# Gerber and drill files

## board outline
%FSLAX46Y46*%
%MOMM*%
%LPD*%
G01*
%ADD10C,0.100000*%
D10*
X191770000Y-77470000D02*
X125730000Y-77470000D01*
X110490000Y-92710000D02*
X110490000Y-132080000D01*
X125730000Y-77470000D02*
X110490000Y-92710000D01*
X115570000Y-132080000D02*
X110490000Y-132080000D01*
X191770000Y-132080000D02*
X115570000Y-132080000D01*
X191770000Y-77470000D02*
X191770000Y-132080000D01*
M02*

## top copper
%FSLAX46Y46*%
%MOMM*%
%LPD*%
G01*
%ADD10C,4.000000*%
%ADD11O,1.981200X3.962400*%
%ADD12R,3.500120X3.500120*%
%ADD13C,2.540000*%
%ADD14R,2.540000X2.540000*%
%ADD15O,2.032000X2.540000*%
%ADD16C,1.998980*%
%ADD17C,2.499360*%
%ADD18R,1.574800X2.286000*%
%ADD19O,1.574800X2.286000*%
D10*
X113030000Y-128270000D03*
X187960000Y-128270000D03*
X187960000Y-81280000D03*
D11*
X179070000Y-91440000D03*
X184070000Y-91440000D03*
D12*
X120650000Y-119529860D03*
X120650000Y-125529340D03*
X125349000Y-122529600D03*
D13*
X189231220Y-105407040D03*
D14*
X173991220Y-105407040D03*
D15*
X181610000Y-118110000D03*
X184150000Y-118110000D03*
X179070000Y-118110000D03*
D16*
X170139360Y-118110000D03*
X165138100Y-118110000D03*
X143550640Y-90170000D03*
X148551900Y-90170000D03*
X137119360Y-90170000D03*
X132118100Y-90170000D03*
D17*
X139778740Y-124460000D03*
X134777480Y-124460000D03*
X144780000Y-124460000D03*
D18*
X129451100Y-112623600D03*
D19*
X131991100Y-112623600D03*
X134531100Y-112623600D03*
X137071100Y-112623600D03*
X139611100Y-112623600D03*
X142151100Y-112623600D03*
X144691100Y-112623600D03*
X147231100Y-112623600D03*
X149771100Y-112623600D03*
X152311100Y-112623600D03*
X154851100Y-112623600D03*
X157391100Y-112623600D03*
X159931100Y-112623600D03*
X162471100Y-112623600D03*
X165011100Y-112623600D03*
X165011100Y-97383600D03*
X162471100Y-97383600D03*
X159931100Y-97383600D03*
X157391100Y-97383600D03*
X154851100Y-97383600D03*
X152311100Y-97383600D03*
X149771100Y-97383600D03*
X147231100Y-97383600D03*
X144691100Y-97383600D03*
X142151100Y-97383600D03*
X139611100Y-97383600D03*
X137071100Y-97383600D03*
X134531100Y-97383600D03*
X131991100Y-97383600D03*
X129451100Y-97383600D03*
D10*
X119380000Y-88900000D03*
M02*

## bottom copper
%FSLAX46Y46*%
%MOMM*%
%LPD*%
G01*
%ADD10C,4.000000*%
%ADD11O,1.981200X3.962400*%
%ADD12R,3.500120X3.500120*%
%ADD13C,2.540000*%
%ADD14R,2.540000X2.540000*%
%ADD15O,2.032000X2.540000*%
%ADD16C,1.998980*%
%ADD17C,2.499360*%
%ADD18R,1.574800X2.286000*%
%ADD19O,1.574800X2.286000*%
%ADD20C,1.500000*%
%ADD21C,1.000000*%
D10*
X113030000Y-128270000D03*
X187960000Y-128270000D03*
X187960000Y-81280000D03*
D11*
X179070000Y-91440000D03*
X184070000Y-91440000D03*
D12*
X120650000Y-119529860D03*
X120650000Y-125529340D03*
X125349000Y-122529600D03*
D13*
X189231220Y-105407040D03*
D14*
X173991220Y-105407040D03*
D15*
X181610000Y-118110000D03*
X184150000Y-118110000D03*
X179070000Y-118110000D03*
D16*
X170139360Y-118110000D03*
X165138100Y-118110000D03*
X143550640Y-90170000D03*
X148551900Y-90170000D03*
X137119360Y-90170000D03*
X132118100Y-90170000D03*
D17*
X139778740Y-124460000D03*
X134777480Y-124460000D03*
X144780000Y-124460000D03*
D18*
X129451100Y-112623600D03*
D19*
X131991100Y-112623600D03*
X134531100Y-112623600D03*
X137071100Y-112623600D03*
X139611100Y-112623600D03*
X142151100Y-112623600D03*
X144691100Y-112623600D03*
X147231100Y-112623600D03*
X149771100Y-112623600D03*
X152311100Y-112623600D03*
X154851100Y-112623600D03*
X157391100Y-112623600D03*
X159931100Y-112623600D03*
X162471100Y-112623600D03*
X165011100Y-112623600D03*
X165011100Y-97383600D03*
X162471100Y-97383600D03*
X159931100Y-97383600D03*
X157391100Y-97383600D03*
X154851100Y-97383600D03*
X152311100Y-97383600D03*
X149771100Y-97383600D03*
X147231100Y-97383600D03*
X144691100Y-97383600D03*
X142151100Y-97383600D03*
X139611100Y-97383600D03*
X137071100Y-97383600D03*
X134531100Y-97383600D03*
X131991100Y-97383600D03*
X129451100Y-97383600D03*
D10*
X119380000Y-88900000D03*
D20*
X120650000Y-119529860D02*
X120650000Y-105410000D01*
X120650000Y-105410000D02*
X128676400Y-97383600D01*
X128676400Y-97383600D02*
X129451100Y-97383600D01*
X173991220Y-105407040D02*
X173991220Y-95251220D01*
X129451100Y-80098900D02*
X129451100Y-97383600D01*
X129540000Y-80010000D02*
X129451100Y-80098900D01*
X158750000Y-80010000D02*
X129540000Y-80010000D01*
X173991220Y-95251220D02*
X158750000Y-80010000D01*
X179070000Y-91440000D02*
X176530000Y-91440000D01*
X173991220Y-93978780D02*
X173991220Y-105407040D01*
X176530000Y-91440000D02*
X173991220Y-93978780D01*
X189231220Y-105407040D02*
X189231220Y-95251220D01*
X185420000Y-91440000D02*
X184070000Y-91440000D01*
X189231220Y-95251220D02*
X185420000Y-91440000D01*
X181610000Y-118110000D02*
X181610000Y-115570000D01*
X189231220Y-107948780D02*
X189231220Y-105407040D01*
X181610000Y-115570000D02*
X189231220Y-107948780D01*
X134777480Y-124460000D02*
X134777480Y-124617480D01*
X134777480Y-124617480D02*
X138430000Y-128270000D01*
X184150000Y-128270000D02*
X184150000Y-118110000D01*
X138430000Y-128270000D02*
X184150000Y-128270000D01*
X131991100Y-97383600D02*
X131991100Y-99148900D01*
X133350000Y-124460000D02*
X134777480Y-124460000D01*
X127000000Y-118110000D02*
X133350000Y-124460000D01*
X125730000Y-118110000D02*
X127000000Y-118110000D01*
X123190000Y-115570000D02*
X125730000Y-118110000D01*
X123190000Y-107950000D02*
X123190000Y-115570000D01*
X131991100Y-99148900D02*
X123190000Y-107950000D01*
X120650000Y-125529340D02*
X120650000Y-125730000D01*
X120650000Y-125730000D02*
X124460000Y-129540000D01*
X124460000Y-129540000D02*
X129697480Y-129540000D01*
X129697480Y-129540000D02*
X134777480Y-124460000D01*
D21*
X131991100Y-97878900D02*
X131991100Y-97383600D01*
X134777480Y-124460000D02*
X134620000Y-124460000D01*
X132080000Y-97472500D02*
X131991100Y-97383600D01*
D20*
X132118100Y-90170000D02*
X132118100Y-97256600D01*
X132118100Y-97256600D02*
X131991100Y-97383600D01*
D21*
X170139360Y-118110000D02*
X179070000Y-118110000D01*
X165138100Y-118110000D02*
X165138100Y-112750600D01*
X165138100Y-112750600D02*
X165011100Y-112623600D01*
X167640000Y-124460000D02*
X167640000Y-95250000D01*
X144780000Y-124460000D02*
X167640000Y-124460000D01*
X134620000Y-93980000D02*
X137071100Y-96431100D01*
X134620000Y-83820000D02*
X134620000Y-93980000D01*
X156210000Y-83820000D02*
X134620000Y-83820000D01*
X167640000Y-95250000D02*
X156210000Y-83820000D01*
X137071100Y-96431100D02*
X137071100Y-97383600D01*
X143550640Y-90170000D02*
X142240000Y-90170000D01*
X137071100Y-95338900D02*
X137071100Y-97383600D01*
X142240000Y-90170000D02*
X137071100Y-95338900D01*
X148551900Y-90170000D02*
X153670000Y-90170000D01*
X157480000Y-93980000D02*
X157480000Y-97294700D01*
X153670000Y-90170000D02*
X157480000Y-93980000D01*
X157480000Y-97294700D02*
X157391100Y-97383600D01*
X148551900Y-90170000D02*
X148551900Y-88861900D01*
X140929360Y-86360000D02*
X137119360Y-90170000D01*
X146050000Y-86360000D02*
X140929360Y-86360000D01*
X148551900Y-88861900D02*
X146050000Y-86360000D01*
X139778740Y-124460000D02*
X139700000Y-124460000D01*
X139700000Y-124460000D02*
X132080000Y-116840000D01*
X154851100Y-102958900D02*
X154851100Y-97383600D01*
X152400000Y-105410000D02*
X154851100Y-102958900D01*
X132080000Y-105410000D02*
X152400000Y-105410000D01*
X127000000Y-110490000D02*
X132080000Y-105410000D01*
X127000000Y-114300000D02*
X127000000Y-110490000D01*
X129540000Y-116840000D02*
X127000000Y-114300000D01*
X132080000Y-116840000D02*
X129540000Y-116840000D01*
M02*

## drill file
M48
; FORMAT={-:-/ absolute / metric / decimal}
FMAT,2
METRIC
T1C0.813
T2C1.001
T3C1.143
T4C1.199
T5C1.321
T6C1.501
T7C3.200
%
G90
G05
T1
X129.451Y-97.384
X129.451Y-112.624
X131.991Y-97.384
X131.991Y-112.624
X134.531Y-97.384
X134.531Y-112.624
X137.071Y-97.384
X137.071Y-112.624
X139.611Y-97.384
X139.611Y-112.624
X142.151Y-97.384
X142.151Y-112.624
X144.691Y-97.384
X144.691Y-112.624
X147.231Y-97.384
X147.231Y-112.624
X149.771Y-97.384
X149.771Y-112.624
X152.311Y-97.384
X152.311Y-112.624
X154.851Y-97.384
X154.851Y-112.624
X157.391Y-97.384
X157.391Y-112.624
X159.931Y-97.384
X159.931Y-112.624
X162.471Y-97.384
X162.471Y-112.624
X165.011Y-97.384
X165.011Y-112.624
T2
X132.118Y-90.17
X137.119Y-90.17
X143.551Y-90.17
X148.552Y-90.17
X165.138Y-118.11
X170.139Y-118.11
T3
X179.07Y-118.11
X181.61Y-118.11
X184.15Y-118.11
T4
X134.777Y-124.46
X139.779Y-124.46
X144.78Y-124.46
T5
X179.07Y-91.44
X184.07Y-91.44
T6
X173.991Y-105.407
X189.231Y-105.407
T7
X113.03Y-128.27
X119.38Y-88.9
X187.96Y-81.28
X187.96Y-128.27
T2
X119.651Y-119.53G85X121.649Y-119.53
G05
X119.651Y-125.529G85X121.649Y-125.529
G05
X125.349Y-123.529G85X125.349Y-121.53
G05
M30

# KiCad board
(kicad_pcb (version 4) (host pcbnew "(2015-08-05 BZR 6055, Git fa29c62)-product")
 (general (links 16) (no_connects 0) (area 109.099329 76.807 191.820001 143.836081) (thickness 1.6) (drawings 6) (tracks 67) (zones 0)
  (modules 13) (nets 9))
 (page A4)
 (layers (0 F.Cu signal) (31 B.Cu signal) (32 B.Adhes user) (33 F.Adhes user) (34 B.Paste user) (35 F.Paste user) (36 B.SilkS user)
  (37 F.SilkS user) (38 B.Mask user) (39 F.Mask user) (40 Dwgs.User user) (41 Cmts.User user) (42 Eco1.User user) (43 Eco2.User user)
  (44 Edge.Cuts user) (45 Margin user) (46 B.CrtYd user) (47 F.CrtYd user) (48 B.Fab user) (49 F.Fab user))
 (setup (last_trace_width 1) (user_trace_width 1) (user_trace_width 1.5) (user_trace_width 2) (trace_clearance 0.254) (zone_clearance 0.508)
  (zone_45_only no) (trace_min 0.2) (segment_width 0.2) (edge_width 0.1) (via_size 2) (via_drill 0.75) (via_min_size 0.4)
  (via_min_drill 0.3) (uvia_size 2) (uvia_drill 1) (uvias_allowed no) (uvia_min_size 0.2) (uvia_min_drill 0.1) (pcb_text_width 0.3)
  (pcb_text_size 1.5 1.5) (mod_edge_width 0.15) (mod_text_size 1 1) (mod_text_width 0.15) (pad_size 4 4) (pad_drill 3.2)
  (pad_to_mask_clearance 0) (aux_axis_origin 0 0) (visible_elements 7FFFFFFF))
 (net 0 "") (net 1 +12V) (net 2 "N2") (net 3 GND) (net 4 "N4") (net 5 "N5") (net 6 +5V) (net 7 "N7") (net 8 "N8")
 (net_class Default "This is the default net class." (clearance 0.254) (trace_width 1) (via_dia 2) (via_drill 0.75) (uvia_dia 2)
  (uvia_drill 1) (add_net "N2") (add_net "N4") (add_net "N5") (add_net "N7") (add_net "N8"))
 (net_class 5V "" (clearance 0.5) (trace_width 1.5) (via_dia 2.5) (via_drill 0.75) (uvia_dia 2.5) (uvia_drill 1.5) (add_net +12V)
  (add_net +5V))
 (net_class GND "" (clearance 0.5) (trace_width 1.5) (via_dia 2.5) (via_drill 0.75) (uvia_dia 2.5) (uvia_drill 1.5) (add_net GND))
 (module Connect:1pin (layer F.Cu) (at 113.03 128.27)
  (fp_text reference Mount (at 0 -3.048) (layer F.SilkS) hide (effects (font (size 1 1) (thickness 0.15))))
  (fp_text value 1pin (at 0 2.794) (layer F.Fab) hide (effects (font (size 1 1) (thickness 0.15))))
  (pad 1 thru_hole circle (at 0 0) (size 4 4) (drill 3.2) (layers *.Cu *.Mask F.SilkS)))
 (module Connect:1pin (layer F.Cu) (at 187.96 128.27)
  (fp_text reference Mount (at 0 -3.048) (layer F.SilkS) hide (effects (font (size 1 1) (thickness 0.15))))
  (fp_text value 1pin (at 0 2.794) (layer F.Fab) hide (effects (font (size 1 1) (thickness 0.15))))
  (pad 1 thru_hole circle (at 0 0) (size 4 4) (drill 3.2) (layers *.Cu *.Mask F.SilkS)))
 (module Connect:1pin (layer F.Cu) (at 187.96 81.28)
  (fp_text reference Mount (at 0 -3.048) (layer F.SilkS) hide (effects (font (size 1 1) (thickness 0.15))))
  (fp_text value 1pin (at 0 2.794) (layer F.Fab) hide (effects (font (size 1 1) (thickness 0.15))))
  (pad 1 thru_hole circle (at 0 0) (size 4 4) (drill 3.2) (layers *.Cu *.Mask F.SilkS)))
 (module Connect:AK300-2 (layer F.Cu) (at 179.07 91.44)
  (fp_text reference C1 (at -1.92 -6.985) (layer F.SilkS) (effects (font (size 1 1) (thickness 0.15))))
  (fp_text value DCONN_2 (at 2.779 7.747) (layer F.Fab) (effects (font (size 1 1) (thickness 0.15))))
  (pad 1 thru_hole oval (at 0 0) (size 1.9812 3.9624) (drill 1.3208) (layers *.Cu F.Paste F.SilkS F.Mask) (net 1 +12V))
  (pad 2 thru_hole oval (at 5 0) (size 1.9812 3.9624) (drill 1.3208) (layers *.Cu F.Paste F.SilkS F.Mask) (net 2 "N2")))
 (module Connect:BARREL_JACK (layer F.Cu) (at 120.65 125.73 90)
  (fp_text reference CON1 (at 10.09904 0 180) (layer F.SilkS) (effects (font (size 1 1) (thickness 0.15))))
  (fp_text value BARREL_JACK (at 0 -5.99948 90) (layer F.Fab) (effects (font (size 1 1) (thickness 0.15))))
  (pad 1 thru_hole rect (at 6.20014 0 90) (size 3.50012 3.50012) (drill oval 1.00076 2.99974) (layers *.Cu *.Mask F.SilkS) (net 1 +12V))
  (pad 2 thru_hole rect (at 0.20066 0 90) (size 3.50012 3.50012) (drill oval 1.00076 2.99974) (layers *.Cu *.Mask F.SilkS) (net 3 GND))
  (pad 3 thru_hole rect (at 3.2004 4.699 90) (size 3.50012 3.50012) (drill oval 2.99974 1.00076) (layers *.Cu *.Mask F.SilkS)))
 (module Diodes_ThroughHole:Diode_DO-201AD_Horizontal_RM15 (layer F.Cu) (at 173.99 105.41)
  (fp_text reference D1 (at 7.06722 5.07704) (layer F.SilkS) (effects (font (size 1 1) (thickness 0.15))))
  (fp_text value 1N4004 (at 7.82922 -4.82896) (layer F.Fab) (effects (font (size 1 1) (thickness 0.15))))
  (pad 2 thru_hole circle (at 15.24122 -0.00296 180) (size 2.54 2.54) (drill 1.50114) (layers *.Cu *.Mask F.SilkS) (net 2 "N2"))
  (pad 1 thru_hole rect (at 0.00122 -0.00296 180) (size 2.54 2.54) (drill 1.50114) (layers *.Cu *.Mask F.SilkS) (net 1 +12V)))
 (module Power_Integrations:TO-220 (layer F.Cu) (at 181.61 118.11)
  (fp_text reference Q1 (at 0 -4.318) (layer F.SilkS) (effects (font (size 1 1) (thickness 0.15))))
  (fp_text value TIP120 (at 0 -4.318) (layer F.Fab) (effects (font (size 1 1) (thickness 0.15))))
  (pad 2 thru_hole oval (at 0 0) (size 2.032 2.54) (drill 1.143) (layers *.Cu *.Mask F.SilkS) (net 2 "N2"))
  (pad 3 thru_hole oval (at 2.54 0) (size 2.032 2.54) (drill 1.143) (layers *.Cu *.Mask F.SilkS) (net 3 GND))
  (pad 1 thru_hole oval (at -2.54 0) (size 2.032 2.54) (drill 1.143) (layers *.Cu *.Mask F.SilkS) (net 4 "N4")))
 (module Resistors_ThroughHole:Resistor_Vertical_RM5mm (layer F.Cu) (at 167.64 118.11 180)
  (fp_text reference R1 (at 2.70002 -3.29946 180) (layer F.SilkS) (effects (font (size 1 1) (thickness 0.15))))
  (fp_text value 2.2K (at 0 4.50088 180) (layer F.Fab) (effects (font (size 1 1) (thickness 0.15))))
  (pad 1 thru_hole circle (at -2.49936 0 180) (size 1.99898 1.99898) (drill 1.00076) (layers *.Cu *.SilkS *.Mask) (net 4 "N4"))
  (pad 2 thru_hole circle (at 2.5019 0 180) (size 1.99898 1.99898) (drill 1.00076) (layers *.Cu *.SilkS *.Mask) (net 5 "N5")))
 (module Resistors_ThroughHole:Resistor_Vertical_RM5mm (layer F.Cu) (at 146.05 90.17)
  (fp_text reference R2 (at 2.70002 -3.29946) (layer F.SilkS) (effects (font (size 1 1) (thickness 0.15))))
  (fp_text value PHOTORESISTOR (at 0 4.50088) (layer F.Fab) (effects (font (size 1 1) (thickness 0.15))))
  (pad 1 thru_hole circle (at -2.49936 0) (size 1.99898 1.99898) (drill 1.00076) (layers *.Cu *.SilkS *.Mask) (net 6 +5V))
  (pad 2 thru_hole circle (at 2.5019 0) (size 1.99898 1.99898) (drill 1.00076) (layers *.Cu *.SilkS *.Mask) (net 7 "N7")))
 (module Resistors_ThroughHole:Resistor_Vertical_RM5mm (layer F.Cu) (at 134.62 90.17 180)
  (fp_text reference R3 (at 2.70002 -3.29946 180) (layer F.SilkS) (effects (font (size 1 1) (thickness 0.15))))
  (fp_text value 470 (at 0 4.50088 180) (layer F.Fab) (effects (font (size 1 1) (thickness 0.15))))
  (pad 1 thru_hole circle (at -2.49936 0 180) (size 1.99898 1.99898) (drill 1.00076) (layers *.Cu *.SilkS *.Mask) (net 7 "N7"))
  (pad 2 thru_hole circle (at 2.5019 0 180) (size 1.99898 1.99898) (drill 1.00076) (layers *.Cu *.SilkS *.Mask) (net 3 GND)))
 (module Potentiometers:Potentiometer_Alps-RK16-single (layer F.Cu) (at 144.78 124.46 270)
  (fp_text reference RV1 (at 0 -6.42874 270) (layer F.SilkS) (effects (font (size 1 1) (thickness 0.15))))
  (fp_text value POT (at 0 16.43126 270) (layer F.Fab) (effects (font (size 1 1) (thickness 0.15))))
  (pad 2 thru_hole circle (at 0 5.00126 270) (size 2.49936 2.49936) (drill 1.19888) (layers *.Cu *.Mask F.SilkS) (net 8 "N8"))
  (pad 3 thru_hole circle (at 0 10.00252 270) (size 2.49936 2.49936) (drill 1.19888) (layers *.Cu *.Mask F.SilkS) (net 3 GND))
  (pad 1 thru_hole circle (at 0 0 270) (size 2.49936 2.49936) (drill 1.19888) (layers *.Cu *.Mask F.SilkS) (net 6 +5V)))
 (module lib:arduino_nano (layer F.Cu) (at 148.5011 105.0036)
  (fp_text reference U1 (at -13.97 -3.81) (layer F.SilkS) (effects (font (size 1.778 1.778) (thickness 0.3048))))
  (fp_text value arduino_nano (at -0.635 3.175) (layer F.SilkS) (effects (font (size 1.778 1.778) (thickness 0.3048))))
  (pad TX1 thru_hole rect (at -19.05 7.62) (size 1.5748 2.286) (drill 0.8128) (layers *.Cu *.Mask F.SilkS))
  (pad RX0 thru_hole oval (at -16.51 7.62) (size 1.5748 2.286) (drill 0.8128) (layers *.Cu *.Mask F.SilkS))
  (pad RST1 thru_hole oval (at -13.97 7.62) (size 1.5748 2.286) (drill 0.8128) (layers *.Cu *.Mask F.SilkS))
  (pad GND1 thru_hole oval (at -11.43 7.62) (size 1.5748 2.286) (drill 0.8128) (layers *.Cu *.Mask F.SilkS))
  (pad D2 thru_hole oval (at -8.89 7.62) (size 1.5748 2.286) (drill 0.8128) (layers *.Cu *.Mask F.SilkS))
  (pad D3 thru_hole oval (at -6.35 7.62) (size 1.5748 2.286) (drill 0.8128) (layers *.Cu *.Mask F.SilkS))
  (pad D4 thru_hole oval (at -3.81 7.62) (size 1.5748 2.286) (drill 0.8128) (layers *.Cu *.Mask F.SilkS))
  (pad D5 thru_hole oval (at -1.27 7.62) (size 1.5748 2.286) (drill 0.8128) (layers *.Cu *.Mask F.SilkS))
  (pad D6 thru_hole oval (at 1.27 7.62) (size 1.5748 2.286) (drill 0.8128) (layers *.Cu *.Mask F.SilkS))
  (pad D7 thru_hole oval (at 3.81 7.62) (size 1.5748 2.286) (drill 0.8128) (layers *.Cu *.Mask F.SilkS))
  (pad D8 thru_hole oval (at 6.35 7.62) (size 1.5748 2.286) (drill 0.8128) (layers *.Cu *.Mask F.SilkS))
  (pad D9 thru_hole oval (at 8.89 7.62) (size 1.5748 2.286) (drill 0.8128) (layers *.Cu *.Mask F.SilkS))
  (pad D10 thru_hole oval (at 11.43 7.62) (size 1.5748 2.286) (drill 0.8128) (layers *.Cu *.Mask F.SilkS))
  (pad D11 thru_hole oval (at 13.97 7.62) (size 1.5748 2.286) (drill 0.8128) (layers *.Cu *.Mask F.SilkS))
  (pad D12 thru_hole oval (at 16.51 7.62) (size 1.5748 2.286) (drill 0.8128) (layers *.Cu *.Mask F.SilkS) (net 5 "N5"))
  (pad D13 thru_hole oval (at 16.51 -7.62) (size 1.5748 2.286) (drill 0.8128) (layers *.Cu *.Mask F.SilkS))
  (pad 3V3 thru_hole oval (at 13.97 -7.62) (size 1.5748 2.286) (drill 0.8128) (layers *.Cu *.Mask F.SilkS))
  (pad REF thru_hole oval (at 11.43 -7.62) (size 1.5748 2.286) (drill 0.8128) (layers *.Cu *.Mask F.SilkS))
  (pad A0 thru_hole oval (at 8.89 -7.62) (size 1.5748 2.286) (drill 0.8128) (layers *.Cu *.Mask F.SilkS) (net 7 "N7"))
  (pad A1 thru_hole oval (at 6.35 -7.62) (size 1.5748 2.286) (drill 0.8128) (layers *.Cu *.Mask F.SilkS) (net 8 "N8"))
  (pad A2 thru_hole oval (at 3.81 -7.62) (size 1.5748 2.286) (drill 0.8128) (layers *.Cu *.Mask F.SilkS))
  (pad A3 thru_hole oval (at 1.27 -7.62) (size 1.5748 2.286) (drill 0.8128) (layers *.Cu *.Mask F.SilkS))
  (pad A4 thru_hole oval (at -1.27 -7.62) (size 1.5748 2.286) (drill 0.8128) (layers *.Cu *.Mask F.SilkS))
  (pad A5 thru_hole oval (at -3.81 -7.62) (size 1.5748 2.286) (drill 0.8128) (layers *.Cu *.Mask F.SilkS))
  (pad A6 thru_hole oval (at -6.35 -7.62) (size 1.5748 2.286) (drill 0.8128) (layers *.Cu *.Mask F.SilkS))
  (pad A7 thru_hole oval (at -8.89 -7.62) (size 1.5748 2.286) (drill 0.8128) (layers *.Cu *.Mask F.SilkS))
  (pad 5V thru_hole oval (at -11.43 -7.62) (size 1.5748 2.286) (drill 0.8128) (layers *.Cu *.Mask F.SilkS) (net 6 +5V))
  (pad RST thru_hole oval (at -13.97 -7.62) (size 1.5748 2.286) (drill 0.8128) (layers *.Cu *.Mask F.SilkS))
  (pad GND thru_hole oval (at -16.51 -7.62) (size 1.5748 2.286) (drill 0.8128) (layers *.Cu *.Mask F.SilkS) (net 3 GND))
  (pad VIN thru_hole oval (at -19.05 -7.62) (size 1.5748 2.286) (drill 0.8128) (layers *.Cu *.Mask F.SilkS) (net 1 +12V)))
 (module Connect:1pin (layer F.Cu) (at 119.38 88.9)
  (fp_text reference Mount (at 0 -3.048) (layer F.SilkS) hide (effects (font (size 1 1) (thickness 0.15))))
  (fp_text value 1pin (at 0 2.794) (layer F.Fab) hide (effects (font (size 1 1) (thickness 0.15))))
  (pad 1 thru_hole circle (at 0 0) (size 4 4) (drill 3.2) (layers *.Cu *.Mask F.SilkS)))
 (gr_line (start 191.77 77.47) (end 125.73 77.47) (angle 90) (layer Edge.Cuts) (width 0.1))
 (gr_line (start 110.49 92.71) (end 110.49 132.08) (angle 90) (layer Edge.Cuts) (width 0.1))
 (gr_line (start 125.73 77.47) (end 110.49 92.71) (angle 90) (layer Edge.Cuts) (width 0.1))
 (gr_line (start 115.57 132.08) (end 110.49 132.08) (angle 90) (layer Edge.Cuts) (width 0.1))
 (gr_line (start 191.77 132.08) (end 115.57 132.08) (angle 90) (layer Edge.Cuts) (width 0.1))
 (gr_line (start 191.77 77.47) (end 191.77 132.08) (angle 90) (layer Edge.Cuts) (width 0.1))
 (segment (start 120.65 119.52986) (end 120.65 105.41) (width 1.5) (layer B.Cu) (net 1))
 (segment (start 120.65 105.41) (end 128.6764 97.3836) (width 1.5) (layer B.Cu) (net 1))
 (segment (start 128.6764 97.3836) (end 129.4511 97.3836) (width 1.5) (layer B.Cu) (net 1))
 (segment (start 173.99122 105.40704) (end 173.99122 95.25122) (width 1.5) (layer B.Cu) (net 1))
 (segment (start 129.4511 80.0989) (end 129.4511 97.3836) (width 1.5) (layer B.Cu) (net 1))
 (segment (start 129.54 80.01) (end 129.4511 80.0989) (width 1.5) (layer B.Cu) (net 1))
 (segment (start 158.75 80.01) (end 129.54 80.01) (width 1.5) (layer B.Cu) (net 1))
 (segment (start 173.99122 95.25122) (end 158.75 80.01) (width 1.5) (layer B.Cu) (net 1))
 (segment (start 179.07 91.44) (end 176.53 91.44) (width 1.5) (layer B.Cu) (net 1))
 (segment (start 173.99122 93.97878) (end 173.99122 105.40704) (width 1.5) (layer B.Cu) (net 1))
 (segment (start 176.53 91.44) (end 173.99122 93.97878) (width 1.5) (layer B.Cu) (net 1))
 (segment (start 189.23122 105.40704) (end 189.23122 95.25122) (width 1.5) (layer B.Cu) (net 2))
 (segment (start 185.42 91.44) (end 184.07 91.44) (width 1.5) (layer B.Cu) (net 2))
 (segment (start 189.23122 95.25122) (end 185.42 91.44) (width 1.5) (layer B.Cu) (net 2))
 (segment (start 181.61 118.11) (end 181.61 115.57) (width 1.5) (layer B.Cu) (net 2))
 (segment (start 189.23122 107.94878) (end 189.23122 105.40704) (width 1.5) (layer B.Cu) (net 2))
 (segment (start 181.61 115.57) (end 189.23122 107.94878) (width 1.5) (layer B.Cu) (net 2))
 (segment (start 134.77748 124.46) (end 134.77748 124.61748) (width 1.5) (layer B.Cu) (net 3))
 (segment (start 134.77748 124.61748) (end 138.43 128.27) (width 1.5) (layer B.Cu) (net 3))
 (segment (start 184.15 128.27) (end 184.15 118.11) (width 1.5) (layer B.Cu) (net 3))
 (segment (start 138.43 128.27) (end 184.15 128.27) (width 1.5) (layer B.Cu) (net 3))
 (segment (start 131.9911 97.3836) (end 131.9911 99.1489) (width 1.5) (layer B.Cu) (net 3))
 (segment (start 133.35 124.46) (end 134.77748 124.46) (width 1.5) (layer B.Cu) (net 3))
 (segment (start 127 118.11) (end 133.35 124.46) (width 1.5) (layer B.Cu) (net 3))
 (segment (start 125.73 118.11) (end 127 118.11) (width 1.5) (layer B.Cu) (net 3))
 (segment (start 123.19 115.57) (end 125.73 118.11) (width 1.5) (layer B.Cu) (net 3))
 (segment (start 123.19 107.95) (end 123.19 115.57) (width 1.5) (layer B.Cu) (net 3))
 (segment (start 131.9911 99.1489) (end 123.19 107.95) (width 1.5) (layer B.Cu) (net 3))
 (segment (start 120.65 125.52934) (end 120.65 125.73) (width 1.5) (layer B.Cu) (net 3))
 (segment (start 120.65 125.73) (end 124.46 129.54) (width 1.5) (layer B.Cu) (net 3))
 (segment (start 124.46 129.54) (end 129.69748 129.54) (width 1.5) (layer B.Cu) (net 3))
 (segment (start 129.69748 129.54) (end 134.77748 124.46) (width 1.5) (layer B.Cu) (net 3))
 (segment (start 131.9911 97.8789) (end 131.9911 97.3836) (width 1) (layer B.Cu) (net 3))
 (segment (start 134.77748 124.46) (end 134.62 124.46) (width 1) (layer B.Cu) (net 3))
 (segment (start 132.08 97.4725) (end 131.9911 97.3836) (width 1) (layer B.Cu) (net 3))
 (segment (start 132.1181 90.17) (end 132.1181 97.2566) (width 1.5) (layer B.Cu) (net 3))
 (segment (start 132.1181 97.2566) (end 131.9911 97.3836) (width 1.5) (layer B.Cu) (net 3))
 (segment (start 170.13936 118.11) (end 179.07 118.11) (width 1) (layer B.Cu) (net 4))
 (segment (start 165.1381 118.11) (end 165.1381 112.7506) (width 1) (layer B.Cu) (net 5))
 (segment (start 165.1381 112.7506) (end 165.0111 112.6236) (width 1) (layer B.Cu) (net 5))
 (segment (start 167.64 124.46) (end 167.64 95.25) (width 1) (layer B.Cu) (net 6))
 (segment (start 144.78 124.46) (end 167.64 124.46) (width 1) (layer B.Cu) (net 6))
 (segment (start 134.62 93.98) (end 137.0711 96.4311) (width 1) (layer B.Cu) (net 6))
 (segment (start 134.62 83.82) (end 134.62 93.98) (width 1) (layer B.Cu) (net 6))
 (segment (start 156.21 83.82) (end 134.62 83.82) (width 1) (layer B.Cu) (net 6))
 (segment (start 167.64 95.25) (end 156.21 83.82) (width 1) (layer B.Cu) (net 6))
 (segment (start 137.0711 96.4311) (end 137.0711 97.3836) (width 1) (layer B.Cu) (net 6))
 (segment (start 143.55064 90.17) (end 142.24 90.17) (width 1) (layer B.Cu) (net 6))
 (segment (start 137.0711 95.3389) (end 137.0711 97.3836) (width 1) (layer B.Cu) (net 6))
 (segment (start 142.24 90.17) (end 137.0711 95.3389) (width 1) (layer B.Cu) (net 6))
 (segment (start 148.5519 90.17) (end 153.67 90.17) (width 1) (layer B.Cu) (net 7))
 (segment (start 157.48 93.98) (end 157.48 97.2947) (width 1) (layer B.Cu) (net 7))
 (segment (start 153.67 90.17) (end 157.48 93.98) (width 1) (layer B.Cu) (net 7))
 (segment (start 157.48 97.2947) (end 157.3911 97.3836) (width 1) (layer B.Cu) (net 7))
 (segment (start 148.5519 90.17) (end 148.5519 88.8619) (width 1) (layer B.Cu) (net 7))
 (segment (start 140.92936 86.36) (end 137.11936 90.17) (width 1) (layer B.Cu) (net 7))
 (segment (start 146.05 86.36) (end 140.92936 86.36) (width 1) (layer B.Cu) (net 7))
 (segment (start 148.5519 88.8619) (end 146.05 86.36) (width 1) (layer B.Cu) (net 7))
 (segment (start 139.77874 124.46) (end 139.7 124.46) (width 1) (layer B.Cu) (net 8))
 (segment (start 139.7 124.46) (end 132.08 116.84) (width 1) (layer B.Cu) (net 8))
 (segment (start 154.8511 102.9589) (end 154.8511 97.3836) (width 1) (layer B.Cu) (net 8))
 (segment (start 152.4 105.41) (end 154.8511 102.9589) (width 1) (layer B.Cu) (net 8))
 (segment (start 132.08 105.41) (end 152.4 105.41) (width 1) (layer B.Cu) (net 8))
 (segment (start 127 110.49) (end 132.08 105.41) (width 1) (layer B.Cu) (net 8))
 (segment (start 127 114.3) (end 127 110.49) (width 1) (layer B.Cu) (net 8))
 (segment (start 129.54 116.84) (end 127 114.3) (width 1) (layer B.Cu) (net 8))
 (segment (start 132.08 116.84) (end 129.54 116.84) (width 1) (layer B.Cu) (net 8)))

